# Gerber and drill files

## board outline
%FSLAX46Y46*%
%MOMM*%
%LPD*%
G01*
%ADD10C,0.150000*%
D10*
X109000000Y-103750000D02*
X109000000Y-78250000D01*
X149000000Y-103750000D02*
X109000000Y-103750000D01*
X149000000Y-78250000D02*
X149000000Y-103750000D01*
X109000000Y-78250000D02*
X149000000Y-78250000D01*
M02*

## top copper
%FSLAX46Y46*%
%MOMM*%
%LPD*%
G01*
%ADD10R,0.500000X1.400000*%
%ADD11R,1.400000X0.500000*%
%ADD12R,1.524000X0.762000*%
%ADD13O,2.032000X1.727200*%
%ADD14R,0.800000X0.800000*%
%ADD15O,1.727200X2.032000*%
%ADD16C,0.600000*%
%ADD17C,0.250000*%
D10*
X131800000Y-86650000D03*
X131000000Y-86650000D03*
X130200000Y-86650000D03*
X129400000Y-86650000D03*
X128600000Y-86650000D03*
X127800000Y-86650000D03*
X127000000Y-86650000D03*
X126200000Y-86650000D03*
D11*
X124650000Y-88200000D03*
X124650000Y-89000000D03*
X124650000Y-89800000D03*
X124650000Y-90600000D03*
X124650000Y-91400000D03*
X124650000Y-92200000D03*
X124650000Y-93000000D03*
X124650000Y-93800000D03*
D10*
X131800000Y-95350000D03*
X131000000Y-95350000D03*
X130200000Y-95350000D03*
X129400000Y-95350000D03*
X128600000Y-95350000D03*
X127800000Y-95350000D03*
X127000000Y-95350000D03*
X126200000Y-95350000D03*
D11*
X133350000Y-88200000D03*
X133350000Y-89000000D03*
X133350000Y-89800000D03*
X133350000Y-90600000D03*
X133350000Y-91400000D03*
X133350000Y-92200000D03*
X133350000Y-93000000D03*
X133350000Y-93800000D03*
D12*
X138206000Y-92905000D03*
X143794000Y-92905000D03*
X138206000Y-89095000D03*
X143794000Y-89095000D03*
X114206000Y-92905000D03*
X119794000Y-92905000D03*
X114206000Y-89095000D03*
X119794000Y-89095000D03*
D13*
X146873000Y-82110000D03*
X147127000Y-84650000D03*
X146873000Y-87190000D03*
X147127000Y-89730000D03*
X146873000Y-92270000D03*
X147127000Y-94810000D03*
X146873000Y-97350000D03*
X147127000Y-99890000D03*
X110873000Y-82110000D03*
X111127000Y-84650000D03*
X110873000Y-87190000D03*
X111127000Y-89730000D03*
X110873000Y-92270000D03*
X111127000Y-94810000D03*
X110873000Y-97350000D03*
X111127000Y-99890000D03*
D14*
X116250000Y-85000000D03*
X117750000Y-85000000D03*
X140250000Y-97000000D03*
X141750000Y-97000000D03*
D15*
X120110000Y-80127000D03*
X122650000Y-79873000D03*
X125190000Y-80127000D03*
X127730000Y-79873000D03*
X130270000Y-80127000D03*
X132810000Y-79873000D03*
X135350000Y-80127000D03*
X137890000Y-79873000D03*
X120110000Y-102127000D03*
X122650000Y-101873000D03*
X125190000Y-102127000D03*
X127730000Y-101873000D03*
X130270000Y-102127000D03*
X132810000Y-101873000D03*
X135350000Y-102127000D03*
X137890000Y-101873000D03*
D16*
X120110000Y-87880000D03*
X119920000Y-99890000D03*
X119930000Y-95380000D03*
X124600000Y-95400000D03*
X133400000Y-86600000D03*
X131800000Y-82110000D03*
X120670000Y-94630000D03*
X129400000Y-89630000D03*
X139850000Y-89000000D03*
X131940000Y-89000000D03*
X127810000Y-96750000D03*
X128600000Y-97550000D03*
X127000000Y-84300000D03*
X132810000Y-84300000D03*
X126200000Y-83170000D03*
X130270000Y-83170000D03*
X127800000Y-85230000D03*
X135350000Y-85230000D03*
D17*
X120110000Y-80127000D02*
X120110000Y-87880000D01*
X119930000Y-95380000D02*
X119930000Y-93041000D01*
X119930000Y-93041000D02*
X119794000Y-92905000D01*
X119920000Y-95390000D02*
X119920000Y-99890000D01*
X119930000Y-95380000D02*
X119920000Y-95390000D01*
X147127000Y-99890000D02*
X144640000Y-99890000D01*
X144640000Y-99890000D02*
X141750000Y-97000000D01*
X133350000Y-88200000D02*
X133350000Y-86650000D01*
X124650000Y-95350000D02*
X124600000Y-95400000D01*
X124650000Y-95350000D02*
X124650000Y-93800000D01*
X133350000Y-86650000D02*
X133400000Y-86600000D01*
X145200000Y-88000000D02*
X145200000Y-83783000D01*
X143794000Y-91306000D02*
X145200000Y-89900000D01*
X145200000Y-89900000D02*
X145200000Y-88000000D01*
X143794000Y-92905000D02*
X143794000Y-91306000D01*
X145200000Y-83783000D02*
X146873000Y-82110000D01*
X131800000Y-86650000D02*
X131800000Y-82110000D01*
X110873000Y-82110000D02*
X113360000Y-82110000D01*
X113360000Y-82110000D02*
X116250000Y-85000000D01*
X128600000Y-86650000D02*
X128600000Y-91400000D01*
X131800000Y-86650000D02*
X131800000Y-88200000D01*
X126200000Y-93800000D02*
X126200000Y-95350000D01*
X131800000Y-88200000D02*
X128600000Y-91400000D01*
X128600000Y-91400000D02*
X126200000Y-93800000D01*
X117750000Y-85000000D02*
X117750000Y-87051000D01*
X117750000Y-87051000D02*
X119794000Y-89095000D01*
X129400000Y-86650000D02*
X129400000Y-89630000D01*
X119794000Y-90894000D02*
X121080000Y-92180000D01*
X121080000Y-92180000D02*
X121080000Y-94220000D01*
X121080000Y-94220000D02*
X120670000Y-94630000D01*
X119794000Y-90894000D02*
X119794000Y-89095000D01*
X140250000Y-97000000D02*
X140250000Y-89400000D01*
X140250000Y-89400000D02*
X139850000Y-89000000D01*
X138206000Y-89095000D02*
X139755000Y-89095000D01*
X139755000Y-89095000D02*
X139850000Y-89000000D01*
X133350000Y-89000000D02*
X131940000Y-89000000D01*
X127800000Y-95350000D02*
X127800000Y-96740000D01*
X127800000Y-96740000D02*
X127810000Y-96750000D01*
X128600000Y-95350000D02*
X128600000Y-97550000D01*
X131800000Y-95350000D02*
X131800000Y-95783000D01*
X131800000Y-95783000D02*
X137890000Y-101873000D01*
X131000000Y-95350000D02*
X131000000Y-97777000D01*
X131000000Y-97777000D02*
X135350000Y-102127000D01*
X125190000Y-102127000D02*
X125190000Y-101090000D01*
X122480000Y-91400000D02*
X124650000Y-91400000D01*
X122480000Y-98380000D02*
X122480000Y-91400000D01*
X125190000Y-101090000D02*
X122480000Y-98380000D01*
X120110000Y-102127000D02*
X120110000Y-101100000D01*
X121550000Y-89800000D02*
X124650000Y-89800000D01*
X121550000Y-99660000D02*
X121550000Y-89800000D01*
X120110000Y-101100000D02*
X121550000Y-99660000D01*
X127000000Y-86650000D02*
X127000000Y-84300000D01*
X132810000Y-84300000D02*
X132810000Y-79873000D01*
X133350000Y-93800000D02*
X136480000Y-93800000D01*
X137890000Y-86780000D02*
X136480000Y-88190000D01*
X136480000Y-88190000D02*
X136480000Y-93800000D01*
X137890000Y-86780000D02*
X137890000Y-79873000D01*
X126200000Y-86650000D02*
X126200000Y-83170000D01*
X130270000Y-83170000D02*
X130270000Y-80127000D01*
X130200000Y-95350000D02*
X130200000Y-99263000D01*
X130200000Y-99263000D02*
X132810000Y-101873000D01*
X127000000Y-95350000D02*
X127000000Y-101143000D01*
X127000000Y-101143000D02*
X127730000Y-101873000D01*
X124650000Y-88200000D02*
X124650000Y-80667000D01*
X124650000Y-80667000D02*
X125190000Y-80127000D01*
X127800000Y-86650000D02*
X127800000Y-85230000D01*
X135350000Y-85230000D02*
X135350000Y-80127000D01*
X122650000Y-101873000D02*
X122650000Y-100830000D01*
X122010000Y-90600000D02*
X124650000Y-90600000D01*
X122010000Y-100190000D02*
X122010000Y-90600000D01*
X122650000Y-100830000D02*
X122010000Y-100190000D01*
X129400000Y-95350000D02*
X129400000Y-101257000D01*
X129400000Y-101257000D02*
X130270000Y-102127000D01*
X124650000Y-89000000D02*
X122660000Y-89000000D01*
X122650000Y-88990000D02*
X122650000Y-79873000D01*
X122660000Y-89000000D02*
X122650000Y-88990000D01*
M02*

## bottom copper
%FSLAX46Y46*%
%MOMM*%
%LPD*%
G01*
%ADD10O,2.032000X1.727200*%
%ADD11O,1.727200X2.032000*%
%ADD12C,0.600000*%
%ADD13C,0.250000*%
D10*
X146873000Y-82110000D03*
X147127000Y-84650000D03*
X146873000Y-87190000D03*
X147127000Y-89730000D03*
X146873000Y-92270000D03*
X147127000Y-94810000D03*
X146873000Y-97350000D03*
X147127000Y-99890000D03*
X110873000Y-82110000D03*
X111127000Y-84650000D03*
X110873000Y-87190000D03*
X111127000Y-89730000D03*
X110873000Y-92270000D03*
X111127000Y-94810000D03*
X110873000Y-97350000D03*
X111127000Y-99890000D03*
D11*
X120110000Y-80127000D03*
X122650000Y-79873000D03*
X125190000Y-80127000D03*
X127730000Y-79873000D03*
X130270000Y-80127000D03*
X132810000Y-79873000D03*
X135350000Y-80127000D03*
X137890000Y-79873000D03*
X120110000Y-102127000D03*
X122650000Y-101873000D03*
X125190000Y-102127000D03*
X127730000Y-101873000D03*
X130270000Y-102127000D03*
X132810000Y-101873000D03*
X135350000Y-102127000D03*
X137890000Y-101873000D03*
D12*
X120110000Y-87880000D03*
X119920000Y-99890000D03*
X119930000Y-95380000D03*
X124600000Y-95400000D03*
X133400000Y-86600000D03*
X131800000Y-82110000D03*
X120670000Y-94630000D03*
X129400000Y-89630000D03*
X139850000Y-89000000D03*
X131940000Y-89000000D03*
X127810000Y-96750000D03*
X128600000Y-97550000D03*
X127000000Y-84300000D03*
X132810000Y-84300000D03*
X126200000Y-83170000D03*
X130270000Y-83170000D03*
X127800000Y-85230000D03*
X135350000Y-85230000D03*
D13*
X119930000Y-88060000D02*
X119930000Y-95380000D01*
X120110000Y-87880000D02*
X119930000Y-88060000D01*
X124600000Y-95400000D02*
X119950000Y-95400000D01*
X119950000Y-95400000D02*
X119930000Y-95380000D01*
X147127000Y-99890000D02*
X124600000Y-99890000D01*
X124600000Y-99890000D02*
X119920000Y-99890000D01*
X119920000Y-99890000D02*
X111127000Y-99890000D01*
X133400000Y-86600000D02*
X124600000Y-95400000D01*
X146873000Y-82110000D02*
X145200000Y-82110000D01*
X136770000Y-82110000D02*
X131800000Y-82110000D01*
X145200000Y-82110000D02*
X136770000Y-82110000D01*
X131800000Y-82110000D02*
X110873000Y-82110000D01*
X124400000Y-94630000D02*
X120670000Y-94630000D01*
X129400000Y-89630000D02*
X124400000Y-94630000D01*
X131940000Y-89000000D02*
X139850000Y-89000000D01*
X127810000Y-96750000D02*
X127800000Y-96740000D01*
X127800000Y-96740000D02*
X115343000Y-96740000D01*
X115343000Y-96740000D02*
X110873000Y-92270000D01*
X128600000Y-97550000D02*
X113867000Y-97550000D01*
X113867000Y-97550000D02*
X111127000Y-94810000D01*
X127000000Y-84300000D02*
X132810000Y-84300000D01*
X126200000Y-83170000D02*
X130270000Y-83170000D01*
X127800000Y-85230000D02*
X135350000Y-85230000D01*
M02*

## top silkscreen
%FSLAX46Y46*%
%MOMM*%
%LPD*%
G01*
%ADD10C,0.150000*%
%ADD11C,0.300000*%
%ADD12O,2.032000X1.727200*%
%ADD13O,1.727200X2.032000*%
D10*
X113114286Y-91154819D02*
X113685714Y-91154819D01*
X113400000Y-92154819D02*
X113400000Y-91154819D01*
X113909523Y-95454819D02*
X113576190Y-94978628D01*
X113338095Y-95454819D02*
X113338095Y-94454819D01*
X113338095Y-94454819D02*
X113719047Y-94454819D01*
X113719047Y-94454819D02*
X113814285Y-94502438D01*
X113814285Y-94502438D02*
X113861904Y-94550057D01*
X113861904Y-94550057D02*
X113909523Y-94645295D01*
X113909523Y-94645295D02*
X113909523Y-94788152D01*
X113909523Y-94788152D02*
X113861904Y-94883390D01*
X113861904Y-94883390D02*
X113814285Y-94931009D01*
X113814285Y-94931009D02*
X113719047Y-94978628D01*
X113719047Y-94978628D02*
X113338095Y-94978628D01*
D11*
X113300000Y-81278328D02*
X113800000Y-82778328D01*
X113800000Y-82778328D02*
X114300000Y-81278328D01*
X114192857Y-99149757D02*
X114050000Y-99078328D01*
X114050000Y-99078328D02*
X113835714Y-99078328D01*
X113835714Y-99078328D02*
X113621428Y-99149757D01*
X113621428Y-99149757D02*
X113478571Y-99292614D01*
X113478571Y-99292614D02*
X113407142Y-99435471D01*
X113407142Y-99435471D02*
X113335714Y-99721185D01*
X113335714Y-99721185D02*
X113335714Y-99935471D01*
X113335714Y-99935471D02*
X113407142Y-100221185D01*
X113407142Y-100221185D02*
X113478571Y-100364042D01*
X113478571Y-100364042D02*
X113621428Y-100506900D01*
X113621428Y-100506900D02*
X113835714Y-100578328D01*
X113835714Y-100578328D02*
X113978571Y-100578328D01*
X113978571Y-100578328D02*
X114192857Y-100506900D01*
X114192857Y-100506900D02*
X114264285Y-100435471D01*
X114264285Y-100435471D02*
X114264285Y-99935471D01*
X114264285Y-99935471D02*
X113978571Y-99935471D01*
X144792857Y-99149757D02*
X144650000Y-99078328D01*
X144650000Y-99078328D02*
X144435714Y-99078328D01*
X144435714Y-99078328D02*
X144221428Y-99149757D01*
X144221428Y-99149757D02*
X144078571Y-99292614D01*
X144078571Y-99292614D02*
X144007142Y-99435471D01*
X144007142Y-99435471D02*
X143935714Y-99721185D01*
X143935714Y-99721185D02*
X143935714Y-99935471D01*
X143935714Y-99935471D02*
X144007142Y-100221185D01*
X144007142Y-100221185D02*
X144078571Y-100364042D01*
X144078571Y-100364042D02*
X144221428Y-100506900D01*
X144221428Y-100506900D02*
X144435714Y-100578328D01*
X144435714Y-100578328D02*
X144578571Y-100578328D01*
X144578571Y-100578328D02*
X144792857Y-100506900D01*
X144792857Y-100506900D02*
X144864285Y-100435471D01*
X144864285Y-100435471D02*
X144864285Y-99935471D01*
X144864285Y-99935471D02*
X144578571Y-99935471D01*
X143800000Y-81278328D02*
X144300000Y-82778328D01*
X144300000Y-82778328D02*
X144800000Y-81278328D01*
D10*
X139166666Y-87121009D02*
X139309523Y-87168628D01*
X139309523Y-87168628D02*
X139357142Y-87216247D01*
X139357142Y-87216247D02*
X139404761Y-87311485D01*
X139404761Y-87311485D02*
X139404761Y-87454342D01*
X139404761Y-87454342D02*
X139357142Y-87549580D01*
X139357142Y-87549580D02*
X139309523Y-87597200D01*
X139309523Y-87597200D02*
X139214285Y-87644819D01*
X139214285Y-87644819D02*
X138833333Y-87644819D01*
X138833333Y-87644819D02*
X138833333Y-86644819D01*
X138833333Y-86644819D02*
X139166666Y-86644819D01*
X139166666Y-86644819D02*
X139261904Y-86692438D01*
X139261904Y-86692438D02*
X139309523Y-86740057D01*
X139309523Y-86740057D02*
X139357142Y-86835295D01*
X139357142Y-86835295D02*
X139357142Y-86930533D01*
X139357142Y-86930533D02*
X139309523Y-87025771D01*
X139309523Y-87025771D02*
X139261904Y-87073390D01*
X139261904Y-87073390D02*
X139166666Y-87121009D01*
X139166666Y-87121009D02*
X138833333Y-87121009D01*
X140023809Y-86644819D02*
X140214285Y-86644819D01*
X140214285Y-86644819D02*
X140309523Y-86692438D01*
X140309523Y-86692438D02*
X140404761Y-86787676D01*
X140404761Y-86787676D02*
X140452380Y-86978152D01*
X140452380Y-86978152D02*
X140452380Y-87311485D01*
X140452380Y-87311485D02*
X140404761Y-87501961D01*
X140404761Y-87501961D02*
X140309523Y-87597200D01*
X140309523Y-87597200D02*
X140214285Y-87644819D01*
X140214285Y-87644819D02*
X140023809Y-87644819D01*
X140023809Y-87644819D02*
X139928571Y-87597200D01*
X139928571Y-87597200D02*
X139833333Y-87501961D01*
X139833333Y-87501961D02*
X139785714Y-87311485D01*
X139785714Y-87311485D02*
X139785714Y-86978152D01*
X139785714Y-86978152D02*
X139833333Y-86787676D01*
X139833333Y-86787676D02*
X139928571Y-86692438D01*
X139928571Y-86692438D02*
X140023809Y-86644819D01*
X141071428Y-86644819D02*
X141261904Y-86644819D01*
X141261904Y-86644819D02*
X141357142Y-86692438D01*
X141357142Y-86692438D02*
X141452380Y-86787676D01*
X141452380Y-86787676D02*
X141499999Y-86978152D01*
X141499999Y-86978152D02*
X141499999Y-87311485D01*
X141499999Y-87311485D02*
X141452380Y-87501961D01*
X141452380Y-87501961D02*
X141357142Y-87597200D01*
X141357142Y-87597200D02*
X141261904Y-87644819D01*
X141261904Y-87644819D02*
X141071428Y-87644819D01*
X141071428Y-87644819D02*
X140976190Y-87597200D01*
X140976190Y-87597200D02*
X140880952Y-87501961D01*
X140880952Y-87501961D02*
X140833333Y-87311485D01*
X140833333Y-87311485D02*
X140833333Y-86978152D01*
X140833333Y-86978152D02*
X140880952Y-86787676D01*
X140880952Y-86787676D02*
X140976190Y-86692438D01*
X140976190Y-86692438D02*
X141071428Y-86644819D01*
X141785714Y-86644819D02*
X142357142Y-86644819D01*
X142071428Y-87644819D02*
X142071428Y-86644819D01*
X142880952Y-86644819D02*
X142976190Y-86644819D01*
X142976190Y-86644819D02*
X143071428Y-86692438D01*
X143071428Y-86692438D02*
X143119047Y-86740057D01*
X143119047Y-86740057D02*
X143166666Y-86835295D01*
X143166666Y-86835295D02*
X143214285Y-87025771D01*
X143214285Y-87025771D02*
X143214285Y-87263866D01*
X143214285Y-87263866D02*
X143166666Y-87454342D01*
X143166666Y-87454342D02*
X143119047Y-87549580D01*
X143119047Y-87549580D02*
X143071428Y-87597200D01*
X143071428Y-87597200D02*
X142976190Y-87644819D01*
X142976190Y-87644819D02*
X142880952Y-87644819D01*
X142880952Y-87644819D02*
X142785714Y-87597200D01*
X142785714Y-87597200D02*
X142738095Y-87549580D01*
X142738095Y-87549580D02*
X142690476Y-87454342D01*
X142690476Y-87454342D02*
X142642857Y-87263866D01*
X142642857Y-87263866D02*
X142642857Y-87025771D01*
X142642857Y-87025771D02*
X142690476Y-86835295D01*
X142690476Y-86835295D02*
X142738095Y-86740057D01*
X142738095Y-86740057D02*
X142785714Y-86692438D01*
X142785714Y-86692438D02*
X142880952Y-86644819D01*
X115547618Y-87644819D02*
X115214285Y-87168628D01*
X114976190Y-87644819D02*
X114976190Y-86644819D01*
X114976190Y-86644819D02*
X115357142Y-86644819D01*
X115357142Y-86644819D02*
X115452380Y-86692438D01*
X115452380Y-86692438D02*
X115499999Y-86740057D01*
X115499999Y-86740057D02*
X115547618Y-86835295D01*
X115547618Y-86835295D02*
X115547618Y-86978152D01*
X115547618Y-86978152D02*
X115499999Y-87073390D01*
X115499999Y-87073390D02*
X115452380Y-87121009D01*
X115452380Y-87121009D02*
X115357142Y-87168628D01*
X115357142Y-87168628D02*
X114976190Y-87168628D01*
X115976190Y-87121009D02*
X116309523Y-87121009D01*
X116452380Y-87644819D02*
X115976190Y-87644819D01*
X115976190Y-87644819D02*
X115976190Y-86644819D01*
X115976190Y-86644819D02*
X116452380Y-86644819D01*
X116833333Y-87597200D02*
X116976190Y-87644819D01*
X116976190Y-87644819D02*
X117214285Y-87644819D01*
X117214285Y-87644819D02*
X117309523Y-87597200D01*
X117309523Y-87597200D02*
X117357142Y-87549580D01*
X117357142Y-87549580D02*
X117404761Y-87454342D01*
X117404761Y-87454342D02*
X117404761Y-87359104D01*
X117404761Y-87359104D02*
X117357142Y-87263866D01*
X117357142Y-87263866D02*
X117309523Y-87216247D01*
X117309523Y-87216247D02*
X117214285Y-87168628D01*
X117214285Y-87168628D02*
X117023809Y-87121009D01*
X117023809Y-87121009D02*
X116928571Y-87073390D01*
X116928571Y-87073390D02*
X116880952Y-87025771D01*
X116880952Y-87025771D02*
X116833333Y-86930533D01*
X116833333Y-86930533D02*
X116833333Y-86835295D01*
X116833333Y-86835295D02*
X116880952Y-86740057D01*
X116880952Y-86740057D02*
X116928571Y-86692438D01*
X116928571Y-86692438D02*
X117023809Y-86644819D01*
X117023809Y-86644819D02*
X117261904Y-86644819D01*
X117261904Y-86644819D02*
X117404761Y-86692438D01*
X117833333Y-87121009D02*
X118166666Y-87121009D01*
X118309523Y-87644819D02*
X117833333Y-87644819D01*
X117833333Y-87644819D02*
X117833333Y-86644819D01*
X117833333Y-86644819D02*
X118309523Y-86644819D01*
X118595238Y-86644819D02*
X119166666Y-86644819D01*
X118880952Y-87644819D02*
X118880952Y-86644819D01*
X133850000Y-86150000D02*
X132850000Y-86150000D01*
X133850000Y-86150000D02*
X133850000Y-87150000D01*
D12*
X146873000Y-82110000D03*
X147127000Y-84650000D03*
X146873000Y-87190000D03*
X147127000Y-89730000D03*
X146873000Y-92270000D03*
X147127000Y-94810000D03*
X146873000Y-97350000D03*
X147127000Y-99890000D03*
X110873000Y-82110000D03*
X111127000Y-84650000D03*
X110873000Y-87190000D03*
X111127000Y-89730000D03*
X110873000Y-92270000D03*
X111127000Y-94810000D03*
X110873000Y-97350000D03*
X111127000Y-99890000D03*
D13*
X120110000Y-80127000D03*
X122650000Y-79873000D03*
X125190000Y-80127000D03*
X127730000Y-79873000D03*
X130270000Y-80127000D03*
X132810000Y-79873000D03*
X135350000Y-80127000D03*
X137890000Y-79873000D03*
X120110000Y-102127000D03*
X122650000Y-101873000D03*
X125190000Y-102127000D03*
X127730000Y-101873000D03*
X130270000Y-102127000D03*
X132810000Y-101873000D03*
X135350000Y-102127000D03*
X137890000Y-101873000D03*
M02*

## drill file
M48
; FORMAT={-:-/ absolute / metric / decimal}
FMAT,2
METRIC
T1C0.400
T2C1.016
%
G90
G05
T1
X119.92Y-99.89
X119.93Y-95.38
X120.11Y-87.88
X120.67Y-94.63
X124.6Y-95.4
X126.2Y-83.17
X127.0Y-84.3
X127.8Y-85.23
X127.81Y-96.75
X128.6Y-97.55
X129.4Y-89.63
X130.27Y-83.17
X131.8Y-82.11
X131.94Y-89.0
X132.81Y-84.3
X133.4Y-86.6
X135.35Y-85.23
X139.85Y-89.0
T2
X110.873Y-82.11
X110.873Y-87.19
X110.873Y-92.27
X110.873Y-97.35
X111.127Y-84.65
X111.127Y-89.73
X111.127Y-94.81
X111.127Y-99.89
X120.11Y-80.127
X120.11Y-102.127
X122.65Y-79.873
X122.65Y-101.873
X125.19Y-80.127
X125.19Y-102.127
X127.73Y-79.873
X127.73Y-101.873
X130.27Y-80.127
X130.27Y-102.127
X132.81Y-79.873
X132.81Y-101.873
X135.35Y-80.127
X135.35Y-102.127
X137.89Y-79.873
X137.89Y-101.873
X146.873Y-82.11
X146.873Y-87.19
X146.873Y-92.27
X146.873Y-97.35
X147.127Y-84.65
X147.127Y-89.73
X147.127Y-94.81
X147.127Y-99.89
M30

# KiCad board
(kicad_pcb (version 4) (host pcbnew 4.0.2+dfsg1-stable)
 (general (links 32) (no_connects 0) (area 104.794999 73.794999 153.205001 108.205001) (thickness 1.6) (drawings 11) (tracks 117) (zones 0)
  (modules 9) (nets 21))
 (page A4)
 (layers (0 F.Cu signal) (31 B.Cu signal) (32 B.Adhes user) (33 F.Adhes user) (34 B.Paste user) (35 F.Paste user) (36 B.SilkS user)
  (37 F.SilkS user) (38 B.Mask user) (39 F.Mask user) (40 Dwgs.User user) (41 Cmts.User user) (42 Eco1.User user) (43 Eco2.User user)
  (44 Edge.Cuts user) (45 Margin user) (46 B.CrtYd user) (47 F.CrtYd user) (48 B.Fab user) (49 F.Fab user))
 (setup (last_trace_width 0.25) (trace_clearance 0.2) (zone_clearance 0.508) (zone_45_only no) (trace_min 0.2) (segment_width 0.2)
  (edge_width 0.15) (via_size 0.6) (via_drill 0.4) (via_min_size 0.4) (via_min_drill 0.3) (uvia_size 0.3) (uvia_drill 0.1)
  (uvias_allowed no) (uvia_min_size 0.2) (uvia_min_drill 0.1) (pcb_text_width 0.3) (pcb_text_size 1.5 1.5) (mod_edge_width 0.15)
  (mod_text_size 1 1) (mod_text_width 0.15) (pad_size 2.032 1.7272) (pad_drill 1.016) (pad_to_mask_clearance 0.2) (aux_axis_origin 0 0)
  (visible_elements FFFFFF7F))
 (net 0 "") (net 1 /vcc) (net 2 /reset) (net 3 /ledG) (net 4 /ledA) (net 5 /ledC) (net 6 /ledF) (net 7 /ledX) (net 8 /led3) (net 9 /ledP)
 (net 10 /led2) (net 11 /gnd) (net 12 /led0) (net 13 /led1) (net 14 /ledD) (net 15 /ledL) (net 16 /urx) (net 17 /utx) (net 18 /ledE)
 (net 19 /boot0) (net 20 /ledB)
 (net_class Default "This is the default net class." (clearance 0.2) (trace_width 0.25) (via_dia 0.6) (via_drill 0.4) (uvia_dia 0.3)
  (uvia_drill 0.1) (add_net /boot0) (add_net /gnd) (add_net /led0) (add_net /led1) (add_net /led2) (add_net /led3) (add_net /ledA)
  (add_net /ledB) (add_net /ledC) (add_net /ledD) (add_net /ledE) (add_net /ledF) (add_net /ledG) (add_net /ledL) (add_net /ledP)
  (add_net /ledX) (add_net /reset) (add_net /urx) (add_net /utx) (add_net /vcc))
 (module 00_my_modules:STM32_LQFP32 (layer F.Cu) (at 129 91 270)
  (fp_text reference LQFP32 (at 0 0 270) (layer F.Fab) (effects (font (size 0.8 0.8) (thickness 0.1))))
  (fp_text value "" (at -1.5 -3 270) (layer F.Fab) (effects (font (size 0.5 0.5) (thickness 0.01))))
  (fp_line (start -4.85 -4.85) (end -4.85 -3.85) (layer F.SilkS) (width 0.15))
  (fp_line (start -4.85 -4.85) (end -3.85 -4.85) (layer F.SilkS) (width 0.15))
  (pad 3.3 smd rect (at -4.35 -2.8 270) (size 1.4 0.5) (layers F.Cu F.Paste F.Mask) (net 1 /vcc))
  (pad PF0 smd rect (at -4.35 -2 270) (size 1.4 0.5) (layers F.Cu F.Paste F.Mask))
  (pad PF1 smd rect (at -4.35 -1.2 270) (size 1.4 0.5) (layers F.Cu F.Paste F.Mask))
  (pad RST smd rect (at -4.35 -0.4 270) (size 1.4 0.5) (layers F.Cu F.Paste F.Mask) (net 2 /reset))
  (pad 3.3 smd rect (at -4.35 0.4 270) (size 1.4 0.5) (layers F.Cu F.Paste F.Mask) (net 1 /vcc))
  (pad PA0 smd rect (at -4.35 1.2 270) (size 1.4 0.5) (layers F.Cu F.Paste F.Mask) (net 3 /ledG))
  (pad PA1 smd rect (at -4.35 2 270) (size 1.4 0.5) (layers F.Cu F.Paste F.Mask) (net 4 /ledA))
  (pad PA2 smd rect (at -4.35 2.8 270) (size 1.4 0.5) (layers F.Cu F.Paste F.Mask) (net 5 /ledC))
  (pad PA3 smd rect (at -2.8 4.35) (size 1.4 0.5) (layers F.Cu F.Paste F.Mask) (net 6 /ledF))
  (pad PA4 smd rect (at -2 4.35) (size 1.4 0.5) (layers F.Cu F.Paste F.Mask) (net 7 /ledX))
  (pad PA5 smd rect (at -1.2 4.35) (size 1.4 0.5) (layers F.Cu F.Paste F.Mask) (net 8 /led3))
  (pad PA6 smd rect (at -0.4 4.35) (size 1.4 0.5) (layers F.Cu F.Paste F.Mask) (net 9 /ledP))
  (pad PA7 smd rect (at 0.4 4.35) (size 1.4 0.5) (layers F.Cu F.Paste F.Mask) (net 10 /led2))
  (pad PB0 smd rect (at 1.2 4.35) (size 1.4 0.5) (layers F.Cu F.Paste F.Mask))
  (pad PB1 smd rect (at 2 4.35) (size 1.4 0.5) (layers F.Cu F.Paste F.Mask))
  (pad GND smd rect (at 2.8 4.35) (size 1.4 0.5) (layers F.Cu F.Paste F.Mask) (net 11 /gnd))
  (pad PA14 smd rect (at 4.35 -2.8 270) (size 1.4 0.5) (layers F.Cu F.Paste F.Mask) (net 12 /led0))
  (pad PA13 smd rect (at 4.35 -2 270) (size 1.4 0.5) (layers F.Cu F.Paste F.Mask) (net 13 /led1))
  (pad PA12 smd rect (at 4.35 -1.2 270) (size 1.4 0.5) (layers F.Cu F.Paste F.Mask) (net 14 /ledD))
  (pad PA11 smd rect (at 4.35 -0.4 270) (size 1.4 0.5) (layers F.Cu F.Paste F.Mask) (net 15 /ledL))
  (pad PA10 smd rect (at 4.35 0.4 270) (size 1.4 0.5) (layers F.Cu F.Paste F.Mask) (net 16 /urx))
  (pad PA9 smd rect (at 4.35 1.2 270) (size 1.4 0.5) (layers F.Cu F.Paste F.Mask) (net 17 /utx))
  (pad PA8 smd rect (at 4.35 2 270) (size 1.4 0.5) (layers F.Cu F.Paste F.Mask) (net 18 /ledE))
  (pad 3.3 smd rect (at 4.35 2.8 270) (size 1.4 0.5) (layers F.Cu F.Paste F.Mask) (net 1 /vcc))
  (pad GND smd rect (at -2.8 -4.35) (size 1.4 0.5) (layers F.Cu F.Paste F.Mask) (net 11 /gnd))
  (pad BOOT smd rect (at -2 -4.35) (size 1.4 0.5) (layers F.Cu F.Paste F.Mask) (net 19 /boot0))
  (pad PB7 smd rect (at -1.2 -4.35) (size 1.4 0.5) (layers F.Cu F.Paste F.Mask))
  (pad PB6 smd rect (at -0.4 -4.35) (size 1.4 0.5) (layers F.Cu F.Paste F.Mask))
  (pad PB5 smd rect (at 0.4 -4.35) (size 1.4 0.5) (layers F.Cu F.Paste F.Mask))
  (pad PB4 smd rect (at 1.2 -4.35) (size 1.4 0.5) (layers F.Cu F.Paste F.Mask))
  (pad PB3 smd rect (at 2 -4.35) (size 1.4 0.5) (layers F.Cu F.Paste F.Mask))
  (pad PA15 smd rect (at 2.8 -4.35) (size 1.4 0.5) (layers F.Cu F.Paste F.Mask) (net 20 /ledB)))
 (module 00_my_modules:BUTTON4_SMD (layer F.Cu) (at 141 91)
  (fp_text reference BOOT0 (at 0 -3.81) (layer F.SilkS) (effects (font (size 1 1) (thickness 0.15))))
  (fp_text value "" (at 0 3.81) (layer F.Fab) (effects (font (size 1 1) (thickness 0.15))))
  (pad 1 smd rect (at -2.794 1.905) (size 1.524 0.762) (layers F.Cu F.Paste F.Mask))
  (pad 2 smd rect (at 2.794 1.905) (size 1.524 0.762) (layers F.Cu F.Paste F.Mask) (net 1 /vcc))
  (pad 3 smd rect (at -2.794 -1.905) (size 1.524 0.762) (layers F.Cu F.Paste F.Mask) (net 19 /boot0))
  (pad 4 smd rect (at 2.794 -1.905) (size 1.524 0.762) (layers F.Cu F.Paste F.Mask)))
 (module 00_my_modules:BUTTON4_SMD (layer F.Cu) (at 117 91)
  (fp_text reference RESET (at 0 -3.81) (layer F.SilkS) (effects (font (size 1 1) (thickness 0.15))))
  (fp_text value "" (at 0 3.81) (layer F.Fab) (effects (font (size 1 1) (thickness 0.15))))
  (pad 1 smd rect (at -2.794 1.905) (size 1.524 0.762) (layers F.Cu F.Paste F.Mask))
  (pad 2 smd rect (at 2.794 1.905) (size 1.524 0.762) (layers F.Cu F.Paste F.Mask) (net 11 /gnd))
  (pad 3 smd rect (at -2.794 -1.905) (size 1.524 0.762) (layers F.Cu F.Paste F.Mask))
  (pad 4 smd rect (at 2.794 -1.905) (size 1.524 0.762) (layers F.Cu F.Paste F.Mask) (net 2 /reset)))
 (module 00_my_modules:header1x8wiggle (layer F.Cu) (at 147 91)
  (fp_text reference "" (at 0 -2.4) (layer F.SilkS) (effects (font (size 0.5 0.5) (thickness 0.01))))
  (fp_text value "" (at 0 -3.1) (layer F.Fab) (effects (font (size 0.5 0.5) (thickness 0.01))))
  (pad 1 thru_hole oval (at -0.127 -8.89) (size 2.032 1.7272) (drill 1.016) (layers *.Cu *.Mask F.SilkS) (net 1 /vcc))
  (pad 2 thru_hole oval (at 0.127 -6.35) (size 2.032 1.7272) (drill 1.016) (layers *.Cu *.Mask F.SilkS))
  (pad 3 thru_hole oval (at -0.127 -3.81) (size 2.032 1.7272) (drill 1.016) (layers *.Cu *.Mask F.SilkS))
  (pad 4 thru_hole oval (at 0.127 -1.27) (size 2.032 1.7272) (drill 1.016) (layers *.Cu *.Mask F.SilkS))
  (pad 5 thru_hole oval (at -0.127 1.27) (size 2.032 1.7272) (drill 1.016) (layers *.Cu *.Mask F.SilkS))
  (pad 6 thru_hole oval (at 0.127 3.81) (size 2.032 1.7272) (drill 1.016) (layers *.Cu *.Mask F.SilkS))
  (pad 7 thru_hole oval (at -0.127 6.35) (size 2.032 1.7272) (drill 1.016) (layers *.Cu *.Mask F.SilkS))
  (pad 8 thru_hole oval (at 0.127 8.89) (size 2.032 1.7272) (drill 1.016) (layers *.Cu *.Mask F.SilkS) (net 11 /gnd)))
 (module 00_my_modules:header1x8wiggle (layer F.Cu) (at 111 91)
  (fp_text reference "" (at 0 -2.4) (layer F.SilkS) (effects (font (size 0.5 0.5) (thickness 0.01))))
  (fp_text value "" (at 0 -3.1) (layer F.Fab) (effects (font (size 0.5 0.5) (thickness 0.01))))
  (pad 1 thru_hole oval (at -0.127 -8.89) (size 2.032 1.7272) (drill 1.016) (layers *.Cu *.Mask F.SilkS) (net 1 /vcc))
  (pad 2 thru_hole oval (at 0.127 -6.35) (size 2.032 1.7272) (drill 1.016) (layers *.Cu *.Mask F.SilkS))
  (pad 3 thru_hole oval (at -0.127 -3.81) (size 2.032 1.7272) (drill 1.016) (layers *.Cu *.Mask F.SilkS))
  (pad 4 thru_hole oval (at 0.127 -1.27) (size 2.032 1.7272) (drill 1.016) (layers *.Cu *.Mask F.SilkS))
  (pad 5 thru_hole oval (at -0.127 1.27) (size 2.032 1.7272) (drill 1.016) (layers *.Cu *.Mask F.SilkS) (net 17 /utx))
  (pad 6 thru_hole oval (at 0.127 3.81) (size 2.032 1.7272) (drill 1.016) (layers *.Cu *.Mask F.SilkS) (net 16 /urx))
  (pad 7 thru_hole oval (at -0.127 6.35) (size 2.032 1.7272) (drill 1.016) (layers *.Cu *.Mask F.SilkS))
  (pad 8 thru_hole oval (at 0.127 8.89) (size 2.032 1.7272) (drill 1.016) (layers *.Cu *.Mask F.SilkS) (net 11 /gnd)))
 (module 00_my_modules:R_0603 (layer F.Cu) (at 117 85)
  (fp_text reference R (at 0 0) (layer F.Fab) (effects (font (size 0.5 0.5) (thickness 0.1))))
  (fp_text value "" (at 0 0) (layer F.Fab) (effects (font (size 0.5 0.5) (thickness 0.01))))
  (pad 1 smd rect (at -0.75 0) (size 0.8 0.8) (layers F.Cu F.Paste F.Mask) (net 1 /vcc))
  (pad 2 smd rect (at 0.75 0) (size 0.8 0.8) (layers F.Cu F.Paste F.Mask) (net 2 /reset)))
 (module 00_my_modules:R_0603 (layer F.Cu) (at 141 97)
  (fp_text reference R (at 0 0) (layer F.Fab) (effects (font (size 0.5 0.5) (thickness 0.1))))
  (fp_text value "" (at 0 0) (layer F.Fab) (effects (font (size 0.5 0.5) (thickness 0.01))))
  (pad 1 smd rect (at -0.75 0) (size 0.8 0.8) (layers F.Cu F.Paste F.Mask) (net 19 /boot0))
  (pad 2 smd rect (at 0.75 0) (size 0.8 0.8) (layers F.Cu F.Paste F.Mask) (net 11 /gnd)))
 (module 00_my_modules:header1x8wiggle (layer F.Cu) (at 129 80 90)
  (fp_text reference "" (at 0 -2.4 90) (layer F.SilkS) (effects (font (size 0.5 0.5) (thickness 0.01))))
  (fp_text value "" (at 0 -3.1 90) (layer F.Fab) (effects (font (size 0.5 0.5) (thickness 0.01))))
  (pad N thru_hole oval (at -0.127 -8.89 90) (size 2.032 1.7272) (drill 1.016) (layers *.Cu *.Mask F.SilkS) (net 11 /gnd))
  (pad X thru_hole oval (at 0.127 -6.35 90) (size 2.032 1.7272) (drill 1.016) (layers *.Cu *.Mask F.SilkS) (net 7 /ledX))
  (pad F thru_hole oval (at -0.127 -3.81 90) (size 2.032 1.7272) (drill 1.016) (layers *.Cu *.Mask F.SilkS) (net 6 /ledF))
  (pad N thru_hole oval (at 0.127 -1.27 90) (size 2.032 1.7272) (drill 1.016) (layers *.Cu *.Mask F.SilkS))
  (pad C thru_hole oval (at -0.127 1.27 90) (size 2.032 1.7272) (drill 1.016) (layers *.Cu *.Mask F.SilkS) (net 5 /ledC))
  (pad A thru_hole oval (at 0.127 3.81 90) (size 2.032 1.7272) (drill 1.016) (layers *.Cu *.Mask F.SilkS) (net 4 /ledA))
  (pad G thru_hole oval (at -0.127 6.35 90) (size 2.032 1.7272) (drill 1.016) (layers *.Cu *.Mask F.SilkS) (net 3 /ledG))
  (pad B thru_hole oval (at 0.127 8.89 90) (size 2.032 1.7272) (drill 1.016) (layers *.Cu *.Mask F.SilkS) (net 20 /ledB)))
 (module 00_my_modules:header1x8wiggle (layer F.Cu) (at 129 102 90)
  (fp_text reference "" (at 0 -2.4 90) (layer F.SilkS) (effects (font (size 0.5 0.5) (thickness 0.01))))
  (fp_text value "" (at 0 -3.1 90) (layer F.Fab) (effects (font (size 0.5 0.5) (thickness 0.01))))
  (pad 3 thru_hole oval (at -0.127 -8.89 90) (size 2.032 1.7272) (drill 1.016) (layers *.Cu *.Mask F.SilkS) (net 8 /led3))
  (pad P thru_hole oval (at 0.127 -6.35 90) (size 2.032 1.7272) (drill 1.016) (layers *.Cu *.Mask F.SilkS) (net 9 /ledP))
  (pad 2 thru_hole oval (at -0.127 -3.81 90) (size 2.032 1.7272) (drill 1.016) (layers *.Cu *.Mask F.SilkS) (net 10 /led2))
  (pad E thru_hole oval (at 0.127 -1.27 90) (size 2.032 1.7272) (drill 1.016) (layers *.Cu *.Mask F.SilkS) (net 18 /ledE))
  (pad L thru_hole oval (at -0.127 1.27 90) (size 2.032 1.7272) (drill 1.016) (layers *.Cu *.Mask F.SilkS) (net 15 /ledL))
  (pad D thru_hole oval (at 0.127 3.81 90) (size 2.032 1.7272) (drill 1.016) (layers *.Cu *.Mask F.SilkS) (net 14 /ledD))
  (pad 1 thru_hole oval (at -0.127 6.35 90) (size 2.032 1.7272) (drill 1.016) (layers *.Cu *.Mask F.SilkS) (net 13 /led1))
  (pad 0 thru_hole oval (at 0.127 8.89 90) (size 2.032 1.7272) (drill 1.016) (layers *.Cu *.Mask F.SilkS) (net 12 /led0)))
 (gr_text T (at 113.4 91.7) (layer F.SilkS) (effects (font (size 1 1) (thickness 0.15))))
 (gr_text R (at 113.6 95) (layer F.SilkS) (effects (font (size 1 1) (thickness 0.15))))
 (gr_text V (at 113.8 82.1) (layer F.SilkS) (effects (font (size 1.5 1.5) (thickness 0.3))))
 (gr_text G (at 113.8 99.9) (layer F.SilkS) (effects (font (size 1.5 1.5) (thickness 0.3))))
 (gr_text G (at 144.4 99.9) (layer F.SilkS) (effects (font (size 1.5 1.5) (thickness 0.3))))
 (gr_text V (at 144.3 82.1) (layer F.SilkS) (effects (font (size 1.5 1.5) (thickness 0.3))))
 (gr_line (start 109 103.75) (end 109 78.25) (angle 90) (layer Edge.Cuts) (width 0.15))
 (gr_line (start 149 103.75) (end 109 103.75) (angle 90) (layer Edge.Cuts) (width 0.15))
 (gr_line (start 149 78.25) (end 149 103.75) (angle 90) (layer Edge.Cuts) (width 0.15))
 (gr_line (start 109 78.25) (end 149 78.25) (angle 90) (layer Edge.Cuts) (width 0.15))
 (segment (start 120.11 80.127) (end 120.11 87.88) (width 0.25) (layer F.Cu) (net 11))
 (segment (start 119.93 88.06) (end 119.93 95.38) (width 0.25) (layer B.Cu) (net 11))
 (segment (start 120.11 87.88) (end 119.93 88.06) (width 0.25) (layer B.Cu) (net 11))
 (via (at 120.11 87.88) (size 0.6) (drill 0.4) (layers F.Cu B.Cu) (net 11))
 (segment (start 119.93 95.38) (end 119.93 93.041) (width 0.25) (layer F.Cu) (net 11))
 (segment (start 119.93 93.041) (end 119.794 92.905) (width 0.25) (layer F.Cu) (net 11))
 (segment (start 124.6 95.4) (end 119.95 95.4) (width 0.25) (layer B.Cu) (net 11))
 (via (at 119.92 99.89) (size 0.6) (drill 0.4) (layers F.Cu B.Cu) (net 11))
 (segment (start 119.92 95.39) (end 119.92 99.89) (width 0.25) (layer F.Cu) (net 11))
 (segment (start 119.93 95.38) (end 119.92 95.39) (width 0.25) (layer F.Cu) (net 11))
 (via (at 119.93 95.38) (size 0.6) (drill 0.4) (layers F.Cu B.Cu) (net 11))
 (segment (start 119.95 95.4) (end 119.93 95.38) (width 0.25) (layer B.Cu) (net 11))
 (segment (start 147.127 99.89) (end 144.64 99.89) (width 0.25) (layer F.Cu) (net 11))
 (segment (start 144.64 99.89) (end 141.75 97) (width 0.25) (layer F.Cu) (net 11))
 (segment (start 147.127 99.89) (end 124.6 99.89) (width 0.25) (layer B.Cu) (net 11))
 (segment (start 124.6 99.89) (end 119.92 99.89) (width 0.25) (layer B.Cu) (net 11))
 (segment (start 119.92 99.89) (end 111.127 99.89) (width 0.25) (layer B.Cu) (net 11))
 (segment (start 133.35 88.2) (end 133.35 86.65) (width 0.25) (layer F.Cu) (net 11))
 (segment (start 124.65 95.35) (end 124.6 95.4) (width 0.25) (layer F.Cu) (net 11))
 (via (at 124.6 95.4) (size 0.6) (drill 0.4) (layers F.Cu B.Cu) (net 11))
 (segment (start 124.65 95.35) (end 124.65 93.8) (width 0.25) (layer F.Cu) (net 11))
 (segment (start 133.4 86.6) (end 124.6 95.4) (width 0.25) (layer B.Cu) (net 11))
 (via (at 133.4 86.6) (size 0.6) (drill 0.4) (layers F.Cu B.Cu) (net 11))
 (segment (start 133.35 86.65) (end 133.4 86.6) (width 0.25) (layer F.Cu) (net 11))
 (segment (start 145.2 88) (end 145.2 83.783) (width 0.25) (layer F.Cu) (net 1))
 (segment (start 143.794 91.306) (end 145.2 89.9) (width 0.25) (layer F.Cu) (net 1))
 (segment (start 145.2 89.9) (end 145.2 88) (width 0.25) (layer F.Cu) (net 1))
 (segment (start 143.794 92.905) (end 143.794 91.306) (width 0.25) (layer F.Cu) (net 1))
 (segment (start 145.2 83.783) (end 146.873 82.11) (width 0.25) (layer F.Cu) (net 1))
 (segment (start 131.8 86.65) (end 131.8 82.11) (width 0.25) (layer F.Cu) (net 1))
 (via (at 131.8 82.11) (size 0.6) (drill 0.4) (layers F.Cu B.Cu) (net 1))
 (segment (start 110.873 82.11) (end 113.36 82.11) (width 0.25) (layer F.Cu) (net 1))
 (segment (start 113.36 82.11) (end 116.25 85) (width 0.25) (layer F.Cu) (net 1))
 (segment (start 146.873 82.11) (end 145.2 82.11) (width 0.25) (layer B.Cu) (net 1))
 (segment (start 136.77 82.11) (end 131.8 82.11) (width 0.25) (layer B.Cu) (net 1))
 (segment (start 145.2 82.11) (end 136.77 82.11) (width 0.25) (layer B.Cu) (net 1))
 (segment (start 131.8 82.11) (end 110.873 82.11) (width 0.25) (layer B.Cu) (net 1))
 (segment (start 128.6 86.65) (end 128.6 91.4) (width 0.25) (layer F.Cu) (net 1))
 (segment (start 131.8 86.65) (end 131.8 88.2) (width 0.25) (layer F.Cu) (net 1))
 (segment (start 126.2 93.8) (end 126.2 95.35) (width 0.25) (layer F.Cu) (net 1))
 (segment (start 131.8 88.2) (end 128.6 91.4) (width 0.25) (layer F.Cu) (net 1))
 (segment (start 128.6 91.4) (end 126.2 93.8) (width 0.25) (layer F.Cu) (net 1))
 (segment (start 117.75 85) (end 117.75 87.051) (width 0.25) (layer F.Cu) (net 2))
 (segment (start 117.75 87.051) (end 119.794 89.095) (width 0.25) (layer F.Cu) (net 2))
 (segment (start 129.4 86.65) (end 129.4 89.63) (width 0.25) (layer F.Cu) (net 2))
 (segment (start 119.794 90.894) (end 121.08 92.18) (width 0.25) (layer F.Cu) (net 2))
 (segment (start 121.08 92.18) (end 121.08 94.22) (width 0.25) (layer F.Cu) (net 2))
 (segment (start 121.08 94.22) (end 120.67 94.63) (width 0.25) (layer F.Cu) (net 2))
 (segment (start 119.794 90.894) (end 119.794 89.095) (width 0.25) (layer F.Cu) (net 2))
 (via (at 120.67 94.63) (size 0.6) (drill 0.4) (layers F.Cu B.Cu) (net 2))
 (segment (start 124.4 94.63) (end 120.67 94.63) (width 0.25) (layer B.Cu) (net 2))
 (segment (start 129.4 89.63) (end 124.4 94.63) (width 0.25) (layer B.Cu) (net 2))
 (via (at 129.4 89.63) (size 0.6) (drill 0.4) (layers F.Cu B.Cu) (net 2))
 (segment (start 140.25 97) (end 140.25 89.4) (width 0.25) (layer F.Cu) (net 19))
 (segment (start 140.25 89.4) (end 139.85 89) (width 0.25) (layer F.Cu) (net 19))
 (via (at 139.85 89) (size 0.6) (drill 0.4) (layers F.Cu B.Cu) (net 19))
 (segment (start 138.206 89.095) (end 139.755 89.095) (width 0.25) (layer F.Cu) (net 19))
 (segment (start 139.755 89.095) (end 139.85 89) (width 0.25) (layer F.Cu) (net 19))
 (segment (start 133.35 89) (end 131.94 89) (width 0.25) (layer F.Cu) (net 19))
 (segment (start 131.94 89) (end 139.85 89) (width 0.25) (layer B.Cu) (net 19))
 (via (at 131.94 89) (size 0.6) (drill 0.4) (layers F.Cu B.Cu) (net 19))
 (segment (start 127.8 95.35) (end 127.8 96.74) (width 0.25) (layer F.Cu) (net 17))
 (segment (start 127.8 96.74) (end 127.81 96.75) (width 0.25) (layer F.Cu) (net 17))
 (via (at 127.81 96.75) (size 0.6) (drill 0.4) (layers F.Cu B.Cu) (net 17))
 (segment (start 127.81 96.75) (end 127.8 96.74) (width 0.25) (layer B.Cu) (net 17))
 (segment (start 127.8 96.74) (end 115.343 96.74) (width 0.25) (layer B.Cu) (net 17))
 (segment (start 115.343 96.74) (end 110.873 92.27) (width 0.25) (layer B.Cu) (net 17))
 (segment (start 128.6 97.55) (end 113.867 97.55) (width 0.25) (layer B.Cu) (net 16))
 (via (at 128.6 97.55) (size 0.6) (drill 0.4) (layers F.Cu B.Cu) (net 16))
 (segment (start 128.6 95.35) (end 128.6 97.55) (width 0.25) (layer F.Cu) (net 16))
 (segment (start 113.867 97.55) (end 111.127 94.81) (width 0.25) (layer B.Cu) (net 16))
 (segment (start 131.8 95.35) (end 131.8 95.783) (width 0.25) (layer F.Cu) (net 12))
 (segment (start 131.8 95.783) (end 137.89 101.873) (width 0.25) (layer F.Cu) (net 12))
 (segment (start 131 95.35) (end 131 97.777) (width 0.25) (layer F.Cu) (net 13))
 (segment (start 131 97.777) (end 135.35 102.127) (width 0.25) (layer F.Cu) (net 13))
 (segment (start 125.19 102.127) (end 125.19 101.09) (width 0.25) (layer F.Cu) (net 10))
 (segment (start 122.48 91.4) (end 124.65 91.4) (width 0.25) (layer F.Cu) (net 10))
 (segment (start 122.48 98.38) (end 122.48 91.4) (width 0.25) (layer F.Cu) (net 10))
 (segment (start 125.19 101.09) (end 122.48 98.38) (width 0.25) (layer F.Cu) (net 10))
 (segment (start 120.11 102.127) (end 120.11 101.1) (width 0.25) (layer F.Cu) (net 8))
 (segment (start 121.55 89.8) (end 124.65 89.8) (width 0.25) (layer F.Cu) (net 8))
 (segment (start 121.55 99.66) (end 121.55 89.8) (width 0.25) (layer F.Cu) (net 8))
 (segment (start 120.11 101.1) (end 121.55 99.66) (width 0.25) (layer F.Cu) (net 8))
 (segment (start 127 84.3) (end 132.81 84.3) (width 0.25) (layer B.Cu) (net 4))
 (via (at 127 84.3) (size 0.6) (drill 0.4) (layers F.Cu B.Cu) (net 4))
 (segment (start 127 86.65) (end 127 84.3) (width 0.25) (layer F.Cu) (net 4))
 (segment (start 132.81 84.3) (end 132.81 79.873) (width 0.25) (layer F.Cu) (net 4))
 (via (at 132.81 84.3) (size 0.6) (drill 0.4) (layers F.Cu B.Cu) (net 4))
 (segment (start 133.35 93.8) (end 136.48 93.8) (width 0.25) (layer F.Cu) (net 20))
 (segment (start 137.89 86.78) (end 136.48 88.19) (width 0.25) (layer F.Cu) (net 20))
 (segment (start 136.48 88.19) (end 136.48 93.8) (width 0.25) (layer F.Cu) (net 20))
 (segment (start 137.89 86.78) (end 137.89 79.873) (width 0.25) (layer F.Cu) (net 20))
 (segment (start 126.2 83.17) (end 130.27 83.17) (width 0.25) (layer B.Cu) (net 5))
 (via (at 126.2 83.17) (size 0.6) (drill 0.4) (layers F.Cu B.Cu) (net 5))
 (segment (start 126.2 86.65) (end 126.2 83.17) (width 0.25) (layer F.Cu) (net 5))
 (segment (start 130.27 83.17) (end 130.27 80.127) (width 0.25) (layer F.Cu) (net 5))
 (via (at 130.27 83.17) (size 0.6) (drill 0.4) (layers F.Cu B.Cu) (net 5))
 (segment (start 130.2 95.35) (end 130.2 99.263) (width 0.25) (layer F.Cu) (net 14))
 (segment (start 130.2 99.263) (end 132.81 101.873) (width 0.25) (layer F.Cu) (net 14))
 (segment (start 127 95.35) (end 127 101.143) (width 0.25) (layer F.Cu) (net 18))
 (segment (start 127 101.143) (end 127.73 101.873) (width 0.25) (layer F.Cu) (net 18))
 (segment (start 124.65 88.2) (end 124.65 80.667) (width 0.25) (layer F.Cu) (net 6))
 (segment (start 124.65 80.667) (end 125.19 80.127) (width 0.25) (layer F.Cu) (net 6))
 (segment (start 127.8 85.23) (end 135.35 85.23) (width 0.25) (layer B.Cu) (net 3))
 (via (at 127.8 85.23) (size 0.6) (drill 0.4) (layers F.Cu B.Cu) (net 3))
 (segment (start 127.8 86.65) (end 127.8 85.23) (width 0.25) (layer F.Cu) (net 3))
 (segment (start 135.35 85.23) (end 135.35 80.127) (width 0.25) (layer F.Cu) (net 3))
 (via (at 135.35 85.23) (size 0.6) (drill 0.4) (layers F.Cu B.Cu) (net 3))
 (segment (start 122.65 101.873) (end 122.65 100.83) (width 0.25) (layer F.Cu) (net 9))
 (segment (start 122.01 90.6) (end 124.65 90.6) (width 0.25) (layer F.Cu) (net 9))
 (segment (start 122.01 100.19) (end 122.01 90.6) (width 0.25) (layer F.Cu) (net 9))
 (segment (start 122.65 100.83) (end 122.01 100.19) (width 0.25) (layer F.Cu) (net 9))
 (segment (start 129.4 95.35) (end 129.4 101.257) (width 0.25) (layer F.Cu) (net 15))
 (segment (start 129.4 101.257) (end 130.27 102.127) (width 0.25) (layer F.Cu) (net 15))
 (segment (start 124.65 89) (end 122.66 89) (width 0.25) (layer F.Cu) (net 7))
 (segment (start 122.65 88.99) (end 122.65 79.873) (width 0.25) (layer F.Cu) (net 7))
 (segment (start 122.66 89) (end 122.65 88.99) (width 0.25) (layer F.Cu) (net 7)))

